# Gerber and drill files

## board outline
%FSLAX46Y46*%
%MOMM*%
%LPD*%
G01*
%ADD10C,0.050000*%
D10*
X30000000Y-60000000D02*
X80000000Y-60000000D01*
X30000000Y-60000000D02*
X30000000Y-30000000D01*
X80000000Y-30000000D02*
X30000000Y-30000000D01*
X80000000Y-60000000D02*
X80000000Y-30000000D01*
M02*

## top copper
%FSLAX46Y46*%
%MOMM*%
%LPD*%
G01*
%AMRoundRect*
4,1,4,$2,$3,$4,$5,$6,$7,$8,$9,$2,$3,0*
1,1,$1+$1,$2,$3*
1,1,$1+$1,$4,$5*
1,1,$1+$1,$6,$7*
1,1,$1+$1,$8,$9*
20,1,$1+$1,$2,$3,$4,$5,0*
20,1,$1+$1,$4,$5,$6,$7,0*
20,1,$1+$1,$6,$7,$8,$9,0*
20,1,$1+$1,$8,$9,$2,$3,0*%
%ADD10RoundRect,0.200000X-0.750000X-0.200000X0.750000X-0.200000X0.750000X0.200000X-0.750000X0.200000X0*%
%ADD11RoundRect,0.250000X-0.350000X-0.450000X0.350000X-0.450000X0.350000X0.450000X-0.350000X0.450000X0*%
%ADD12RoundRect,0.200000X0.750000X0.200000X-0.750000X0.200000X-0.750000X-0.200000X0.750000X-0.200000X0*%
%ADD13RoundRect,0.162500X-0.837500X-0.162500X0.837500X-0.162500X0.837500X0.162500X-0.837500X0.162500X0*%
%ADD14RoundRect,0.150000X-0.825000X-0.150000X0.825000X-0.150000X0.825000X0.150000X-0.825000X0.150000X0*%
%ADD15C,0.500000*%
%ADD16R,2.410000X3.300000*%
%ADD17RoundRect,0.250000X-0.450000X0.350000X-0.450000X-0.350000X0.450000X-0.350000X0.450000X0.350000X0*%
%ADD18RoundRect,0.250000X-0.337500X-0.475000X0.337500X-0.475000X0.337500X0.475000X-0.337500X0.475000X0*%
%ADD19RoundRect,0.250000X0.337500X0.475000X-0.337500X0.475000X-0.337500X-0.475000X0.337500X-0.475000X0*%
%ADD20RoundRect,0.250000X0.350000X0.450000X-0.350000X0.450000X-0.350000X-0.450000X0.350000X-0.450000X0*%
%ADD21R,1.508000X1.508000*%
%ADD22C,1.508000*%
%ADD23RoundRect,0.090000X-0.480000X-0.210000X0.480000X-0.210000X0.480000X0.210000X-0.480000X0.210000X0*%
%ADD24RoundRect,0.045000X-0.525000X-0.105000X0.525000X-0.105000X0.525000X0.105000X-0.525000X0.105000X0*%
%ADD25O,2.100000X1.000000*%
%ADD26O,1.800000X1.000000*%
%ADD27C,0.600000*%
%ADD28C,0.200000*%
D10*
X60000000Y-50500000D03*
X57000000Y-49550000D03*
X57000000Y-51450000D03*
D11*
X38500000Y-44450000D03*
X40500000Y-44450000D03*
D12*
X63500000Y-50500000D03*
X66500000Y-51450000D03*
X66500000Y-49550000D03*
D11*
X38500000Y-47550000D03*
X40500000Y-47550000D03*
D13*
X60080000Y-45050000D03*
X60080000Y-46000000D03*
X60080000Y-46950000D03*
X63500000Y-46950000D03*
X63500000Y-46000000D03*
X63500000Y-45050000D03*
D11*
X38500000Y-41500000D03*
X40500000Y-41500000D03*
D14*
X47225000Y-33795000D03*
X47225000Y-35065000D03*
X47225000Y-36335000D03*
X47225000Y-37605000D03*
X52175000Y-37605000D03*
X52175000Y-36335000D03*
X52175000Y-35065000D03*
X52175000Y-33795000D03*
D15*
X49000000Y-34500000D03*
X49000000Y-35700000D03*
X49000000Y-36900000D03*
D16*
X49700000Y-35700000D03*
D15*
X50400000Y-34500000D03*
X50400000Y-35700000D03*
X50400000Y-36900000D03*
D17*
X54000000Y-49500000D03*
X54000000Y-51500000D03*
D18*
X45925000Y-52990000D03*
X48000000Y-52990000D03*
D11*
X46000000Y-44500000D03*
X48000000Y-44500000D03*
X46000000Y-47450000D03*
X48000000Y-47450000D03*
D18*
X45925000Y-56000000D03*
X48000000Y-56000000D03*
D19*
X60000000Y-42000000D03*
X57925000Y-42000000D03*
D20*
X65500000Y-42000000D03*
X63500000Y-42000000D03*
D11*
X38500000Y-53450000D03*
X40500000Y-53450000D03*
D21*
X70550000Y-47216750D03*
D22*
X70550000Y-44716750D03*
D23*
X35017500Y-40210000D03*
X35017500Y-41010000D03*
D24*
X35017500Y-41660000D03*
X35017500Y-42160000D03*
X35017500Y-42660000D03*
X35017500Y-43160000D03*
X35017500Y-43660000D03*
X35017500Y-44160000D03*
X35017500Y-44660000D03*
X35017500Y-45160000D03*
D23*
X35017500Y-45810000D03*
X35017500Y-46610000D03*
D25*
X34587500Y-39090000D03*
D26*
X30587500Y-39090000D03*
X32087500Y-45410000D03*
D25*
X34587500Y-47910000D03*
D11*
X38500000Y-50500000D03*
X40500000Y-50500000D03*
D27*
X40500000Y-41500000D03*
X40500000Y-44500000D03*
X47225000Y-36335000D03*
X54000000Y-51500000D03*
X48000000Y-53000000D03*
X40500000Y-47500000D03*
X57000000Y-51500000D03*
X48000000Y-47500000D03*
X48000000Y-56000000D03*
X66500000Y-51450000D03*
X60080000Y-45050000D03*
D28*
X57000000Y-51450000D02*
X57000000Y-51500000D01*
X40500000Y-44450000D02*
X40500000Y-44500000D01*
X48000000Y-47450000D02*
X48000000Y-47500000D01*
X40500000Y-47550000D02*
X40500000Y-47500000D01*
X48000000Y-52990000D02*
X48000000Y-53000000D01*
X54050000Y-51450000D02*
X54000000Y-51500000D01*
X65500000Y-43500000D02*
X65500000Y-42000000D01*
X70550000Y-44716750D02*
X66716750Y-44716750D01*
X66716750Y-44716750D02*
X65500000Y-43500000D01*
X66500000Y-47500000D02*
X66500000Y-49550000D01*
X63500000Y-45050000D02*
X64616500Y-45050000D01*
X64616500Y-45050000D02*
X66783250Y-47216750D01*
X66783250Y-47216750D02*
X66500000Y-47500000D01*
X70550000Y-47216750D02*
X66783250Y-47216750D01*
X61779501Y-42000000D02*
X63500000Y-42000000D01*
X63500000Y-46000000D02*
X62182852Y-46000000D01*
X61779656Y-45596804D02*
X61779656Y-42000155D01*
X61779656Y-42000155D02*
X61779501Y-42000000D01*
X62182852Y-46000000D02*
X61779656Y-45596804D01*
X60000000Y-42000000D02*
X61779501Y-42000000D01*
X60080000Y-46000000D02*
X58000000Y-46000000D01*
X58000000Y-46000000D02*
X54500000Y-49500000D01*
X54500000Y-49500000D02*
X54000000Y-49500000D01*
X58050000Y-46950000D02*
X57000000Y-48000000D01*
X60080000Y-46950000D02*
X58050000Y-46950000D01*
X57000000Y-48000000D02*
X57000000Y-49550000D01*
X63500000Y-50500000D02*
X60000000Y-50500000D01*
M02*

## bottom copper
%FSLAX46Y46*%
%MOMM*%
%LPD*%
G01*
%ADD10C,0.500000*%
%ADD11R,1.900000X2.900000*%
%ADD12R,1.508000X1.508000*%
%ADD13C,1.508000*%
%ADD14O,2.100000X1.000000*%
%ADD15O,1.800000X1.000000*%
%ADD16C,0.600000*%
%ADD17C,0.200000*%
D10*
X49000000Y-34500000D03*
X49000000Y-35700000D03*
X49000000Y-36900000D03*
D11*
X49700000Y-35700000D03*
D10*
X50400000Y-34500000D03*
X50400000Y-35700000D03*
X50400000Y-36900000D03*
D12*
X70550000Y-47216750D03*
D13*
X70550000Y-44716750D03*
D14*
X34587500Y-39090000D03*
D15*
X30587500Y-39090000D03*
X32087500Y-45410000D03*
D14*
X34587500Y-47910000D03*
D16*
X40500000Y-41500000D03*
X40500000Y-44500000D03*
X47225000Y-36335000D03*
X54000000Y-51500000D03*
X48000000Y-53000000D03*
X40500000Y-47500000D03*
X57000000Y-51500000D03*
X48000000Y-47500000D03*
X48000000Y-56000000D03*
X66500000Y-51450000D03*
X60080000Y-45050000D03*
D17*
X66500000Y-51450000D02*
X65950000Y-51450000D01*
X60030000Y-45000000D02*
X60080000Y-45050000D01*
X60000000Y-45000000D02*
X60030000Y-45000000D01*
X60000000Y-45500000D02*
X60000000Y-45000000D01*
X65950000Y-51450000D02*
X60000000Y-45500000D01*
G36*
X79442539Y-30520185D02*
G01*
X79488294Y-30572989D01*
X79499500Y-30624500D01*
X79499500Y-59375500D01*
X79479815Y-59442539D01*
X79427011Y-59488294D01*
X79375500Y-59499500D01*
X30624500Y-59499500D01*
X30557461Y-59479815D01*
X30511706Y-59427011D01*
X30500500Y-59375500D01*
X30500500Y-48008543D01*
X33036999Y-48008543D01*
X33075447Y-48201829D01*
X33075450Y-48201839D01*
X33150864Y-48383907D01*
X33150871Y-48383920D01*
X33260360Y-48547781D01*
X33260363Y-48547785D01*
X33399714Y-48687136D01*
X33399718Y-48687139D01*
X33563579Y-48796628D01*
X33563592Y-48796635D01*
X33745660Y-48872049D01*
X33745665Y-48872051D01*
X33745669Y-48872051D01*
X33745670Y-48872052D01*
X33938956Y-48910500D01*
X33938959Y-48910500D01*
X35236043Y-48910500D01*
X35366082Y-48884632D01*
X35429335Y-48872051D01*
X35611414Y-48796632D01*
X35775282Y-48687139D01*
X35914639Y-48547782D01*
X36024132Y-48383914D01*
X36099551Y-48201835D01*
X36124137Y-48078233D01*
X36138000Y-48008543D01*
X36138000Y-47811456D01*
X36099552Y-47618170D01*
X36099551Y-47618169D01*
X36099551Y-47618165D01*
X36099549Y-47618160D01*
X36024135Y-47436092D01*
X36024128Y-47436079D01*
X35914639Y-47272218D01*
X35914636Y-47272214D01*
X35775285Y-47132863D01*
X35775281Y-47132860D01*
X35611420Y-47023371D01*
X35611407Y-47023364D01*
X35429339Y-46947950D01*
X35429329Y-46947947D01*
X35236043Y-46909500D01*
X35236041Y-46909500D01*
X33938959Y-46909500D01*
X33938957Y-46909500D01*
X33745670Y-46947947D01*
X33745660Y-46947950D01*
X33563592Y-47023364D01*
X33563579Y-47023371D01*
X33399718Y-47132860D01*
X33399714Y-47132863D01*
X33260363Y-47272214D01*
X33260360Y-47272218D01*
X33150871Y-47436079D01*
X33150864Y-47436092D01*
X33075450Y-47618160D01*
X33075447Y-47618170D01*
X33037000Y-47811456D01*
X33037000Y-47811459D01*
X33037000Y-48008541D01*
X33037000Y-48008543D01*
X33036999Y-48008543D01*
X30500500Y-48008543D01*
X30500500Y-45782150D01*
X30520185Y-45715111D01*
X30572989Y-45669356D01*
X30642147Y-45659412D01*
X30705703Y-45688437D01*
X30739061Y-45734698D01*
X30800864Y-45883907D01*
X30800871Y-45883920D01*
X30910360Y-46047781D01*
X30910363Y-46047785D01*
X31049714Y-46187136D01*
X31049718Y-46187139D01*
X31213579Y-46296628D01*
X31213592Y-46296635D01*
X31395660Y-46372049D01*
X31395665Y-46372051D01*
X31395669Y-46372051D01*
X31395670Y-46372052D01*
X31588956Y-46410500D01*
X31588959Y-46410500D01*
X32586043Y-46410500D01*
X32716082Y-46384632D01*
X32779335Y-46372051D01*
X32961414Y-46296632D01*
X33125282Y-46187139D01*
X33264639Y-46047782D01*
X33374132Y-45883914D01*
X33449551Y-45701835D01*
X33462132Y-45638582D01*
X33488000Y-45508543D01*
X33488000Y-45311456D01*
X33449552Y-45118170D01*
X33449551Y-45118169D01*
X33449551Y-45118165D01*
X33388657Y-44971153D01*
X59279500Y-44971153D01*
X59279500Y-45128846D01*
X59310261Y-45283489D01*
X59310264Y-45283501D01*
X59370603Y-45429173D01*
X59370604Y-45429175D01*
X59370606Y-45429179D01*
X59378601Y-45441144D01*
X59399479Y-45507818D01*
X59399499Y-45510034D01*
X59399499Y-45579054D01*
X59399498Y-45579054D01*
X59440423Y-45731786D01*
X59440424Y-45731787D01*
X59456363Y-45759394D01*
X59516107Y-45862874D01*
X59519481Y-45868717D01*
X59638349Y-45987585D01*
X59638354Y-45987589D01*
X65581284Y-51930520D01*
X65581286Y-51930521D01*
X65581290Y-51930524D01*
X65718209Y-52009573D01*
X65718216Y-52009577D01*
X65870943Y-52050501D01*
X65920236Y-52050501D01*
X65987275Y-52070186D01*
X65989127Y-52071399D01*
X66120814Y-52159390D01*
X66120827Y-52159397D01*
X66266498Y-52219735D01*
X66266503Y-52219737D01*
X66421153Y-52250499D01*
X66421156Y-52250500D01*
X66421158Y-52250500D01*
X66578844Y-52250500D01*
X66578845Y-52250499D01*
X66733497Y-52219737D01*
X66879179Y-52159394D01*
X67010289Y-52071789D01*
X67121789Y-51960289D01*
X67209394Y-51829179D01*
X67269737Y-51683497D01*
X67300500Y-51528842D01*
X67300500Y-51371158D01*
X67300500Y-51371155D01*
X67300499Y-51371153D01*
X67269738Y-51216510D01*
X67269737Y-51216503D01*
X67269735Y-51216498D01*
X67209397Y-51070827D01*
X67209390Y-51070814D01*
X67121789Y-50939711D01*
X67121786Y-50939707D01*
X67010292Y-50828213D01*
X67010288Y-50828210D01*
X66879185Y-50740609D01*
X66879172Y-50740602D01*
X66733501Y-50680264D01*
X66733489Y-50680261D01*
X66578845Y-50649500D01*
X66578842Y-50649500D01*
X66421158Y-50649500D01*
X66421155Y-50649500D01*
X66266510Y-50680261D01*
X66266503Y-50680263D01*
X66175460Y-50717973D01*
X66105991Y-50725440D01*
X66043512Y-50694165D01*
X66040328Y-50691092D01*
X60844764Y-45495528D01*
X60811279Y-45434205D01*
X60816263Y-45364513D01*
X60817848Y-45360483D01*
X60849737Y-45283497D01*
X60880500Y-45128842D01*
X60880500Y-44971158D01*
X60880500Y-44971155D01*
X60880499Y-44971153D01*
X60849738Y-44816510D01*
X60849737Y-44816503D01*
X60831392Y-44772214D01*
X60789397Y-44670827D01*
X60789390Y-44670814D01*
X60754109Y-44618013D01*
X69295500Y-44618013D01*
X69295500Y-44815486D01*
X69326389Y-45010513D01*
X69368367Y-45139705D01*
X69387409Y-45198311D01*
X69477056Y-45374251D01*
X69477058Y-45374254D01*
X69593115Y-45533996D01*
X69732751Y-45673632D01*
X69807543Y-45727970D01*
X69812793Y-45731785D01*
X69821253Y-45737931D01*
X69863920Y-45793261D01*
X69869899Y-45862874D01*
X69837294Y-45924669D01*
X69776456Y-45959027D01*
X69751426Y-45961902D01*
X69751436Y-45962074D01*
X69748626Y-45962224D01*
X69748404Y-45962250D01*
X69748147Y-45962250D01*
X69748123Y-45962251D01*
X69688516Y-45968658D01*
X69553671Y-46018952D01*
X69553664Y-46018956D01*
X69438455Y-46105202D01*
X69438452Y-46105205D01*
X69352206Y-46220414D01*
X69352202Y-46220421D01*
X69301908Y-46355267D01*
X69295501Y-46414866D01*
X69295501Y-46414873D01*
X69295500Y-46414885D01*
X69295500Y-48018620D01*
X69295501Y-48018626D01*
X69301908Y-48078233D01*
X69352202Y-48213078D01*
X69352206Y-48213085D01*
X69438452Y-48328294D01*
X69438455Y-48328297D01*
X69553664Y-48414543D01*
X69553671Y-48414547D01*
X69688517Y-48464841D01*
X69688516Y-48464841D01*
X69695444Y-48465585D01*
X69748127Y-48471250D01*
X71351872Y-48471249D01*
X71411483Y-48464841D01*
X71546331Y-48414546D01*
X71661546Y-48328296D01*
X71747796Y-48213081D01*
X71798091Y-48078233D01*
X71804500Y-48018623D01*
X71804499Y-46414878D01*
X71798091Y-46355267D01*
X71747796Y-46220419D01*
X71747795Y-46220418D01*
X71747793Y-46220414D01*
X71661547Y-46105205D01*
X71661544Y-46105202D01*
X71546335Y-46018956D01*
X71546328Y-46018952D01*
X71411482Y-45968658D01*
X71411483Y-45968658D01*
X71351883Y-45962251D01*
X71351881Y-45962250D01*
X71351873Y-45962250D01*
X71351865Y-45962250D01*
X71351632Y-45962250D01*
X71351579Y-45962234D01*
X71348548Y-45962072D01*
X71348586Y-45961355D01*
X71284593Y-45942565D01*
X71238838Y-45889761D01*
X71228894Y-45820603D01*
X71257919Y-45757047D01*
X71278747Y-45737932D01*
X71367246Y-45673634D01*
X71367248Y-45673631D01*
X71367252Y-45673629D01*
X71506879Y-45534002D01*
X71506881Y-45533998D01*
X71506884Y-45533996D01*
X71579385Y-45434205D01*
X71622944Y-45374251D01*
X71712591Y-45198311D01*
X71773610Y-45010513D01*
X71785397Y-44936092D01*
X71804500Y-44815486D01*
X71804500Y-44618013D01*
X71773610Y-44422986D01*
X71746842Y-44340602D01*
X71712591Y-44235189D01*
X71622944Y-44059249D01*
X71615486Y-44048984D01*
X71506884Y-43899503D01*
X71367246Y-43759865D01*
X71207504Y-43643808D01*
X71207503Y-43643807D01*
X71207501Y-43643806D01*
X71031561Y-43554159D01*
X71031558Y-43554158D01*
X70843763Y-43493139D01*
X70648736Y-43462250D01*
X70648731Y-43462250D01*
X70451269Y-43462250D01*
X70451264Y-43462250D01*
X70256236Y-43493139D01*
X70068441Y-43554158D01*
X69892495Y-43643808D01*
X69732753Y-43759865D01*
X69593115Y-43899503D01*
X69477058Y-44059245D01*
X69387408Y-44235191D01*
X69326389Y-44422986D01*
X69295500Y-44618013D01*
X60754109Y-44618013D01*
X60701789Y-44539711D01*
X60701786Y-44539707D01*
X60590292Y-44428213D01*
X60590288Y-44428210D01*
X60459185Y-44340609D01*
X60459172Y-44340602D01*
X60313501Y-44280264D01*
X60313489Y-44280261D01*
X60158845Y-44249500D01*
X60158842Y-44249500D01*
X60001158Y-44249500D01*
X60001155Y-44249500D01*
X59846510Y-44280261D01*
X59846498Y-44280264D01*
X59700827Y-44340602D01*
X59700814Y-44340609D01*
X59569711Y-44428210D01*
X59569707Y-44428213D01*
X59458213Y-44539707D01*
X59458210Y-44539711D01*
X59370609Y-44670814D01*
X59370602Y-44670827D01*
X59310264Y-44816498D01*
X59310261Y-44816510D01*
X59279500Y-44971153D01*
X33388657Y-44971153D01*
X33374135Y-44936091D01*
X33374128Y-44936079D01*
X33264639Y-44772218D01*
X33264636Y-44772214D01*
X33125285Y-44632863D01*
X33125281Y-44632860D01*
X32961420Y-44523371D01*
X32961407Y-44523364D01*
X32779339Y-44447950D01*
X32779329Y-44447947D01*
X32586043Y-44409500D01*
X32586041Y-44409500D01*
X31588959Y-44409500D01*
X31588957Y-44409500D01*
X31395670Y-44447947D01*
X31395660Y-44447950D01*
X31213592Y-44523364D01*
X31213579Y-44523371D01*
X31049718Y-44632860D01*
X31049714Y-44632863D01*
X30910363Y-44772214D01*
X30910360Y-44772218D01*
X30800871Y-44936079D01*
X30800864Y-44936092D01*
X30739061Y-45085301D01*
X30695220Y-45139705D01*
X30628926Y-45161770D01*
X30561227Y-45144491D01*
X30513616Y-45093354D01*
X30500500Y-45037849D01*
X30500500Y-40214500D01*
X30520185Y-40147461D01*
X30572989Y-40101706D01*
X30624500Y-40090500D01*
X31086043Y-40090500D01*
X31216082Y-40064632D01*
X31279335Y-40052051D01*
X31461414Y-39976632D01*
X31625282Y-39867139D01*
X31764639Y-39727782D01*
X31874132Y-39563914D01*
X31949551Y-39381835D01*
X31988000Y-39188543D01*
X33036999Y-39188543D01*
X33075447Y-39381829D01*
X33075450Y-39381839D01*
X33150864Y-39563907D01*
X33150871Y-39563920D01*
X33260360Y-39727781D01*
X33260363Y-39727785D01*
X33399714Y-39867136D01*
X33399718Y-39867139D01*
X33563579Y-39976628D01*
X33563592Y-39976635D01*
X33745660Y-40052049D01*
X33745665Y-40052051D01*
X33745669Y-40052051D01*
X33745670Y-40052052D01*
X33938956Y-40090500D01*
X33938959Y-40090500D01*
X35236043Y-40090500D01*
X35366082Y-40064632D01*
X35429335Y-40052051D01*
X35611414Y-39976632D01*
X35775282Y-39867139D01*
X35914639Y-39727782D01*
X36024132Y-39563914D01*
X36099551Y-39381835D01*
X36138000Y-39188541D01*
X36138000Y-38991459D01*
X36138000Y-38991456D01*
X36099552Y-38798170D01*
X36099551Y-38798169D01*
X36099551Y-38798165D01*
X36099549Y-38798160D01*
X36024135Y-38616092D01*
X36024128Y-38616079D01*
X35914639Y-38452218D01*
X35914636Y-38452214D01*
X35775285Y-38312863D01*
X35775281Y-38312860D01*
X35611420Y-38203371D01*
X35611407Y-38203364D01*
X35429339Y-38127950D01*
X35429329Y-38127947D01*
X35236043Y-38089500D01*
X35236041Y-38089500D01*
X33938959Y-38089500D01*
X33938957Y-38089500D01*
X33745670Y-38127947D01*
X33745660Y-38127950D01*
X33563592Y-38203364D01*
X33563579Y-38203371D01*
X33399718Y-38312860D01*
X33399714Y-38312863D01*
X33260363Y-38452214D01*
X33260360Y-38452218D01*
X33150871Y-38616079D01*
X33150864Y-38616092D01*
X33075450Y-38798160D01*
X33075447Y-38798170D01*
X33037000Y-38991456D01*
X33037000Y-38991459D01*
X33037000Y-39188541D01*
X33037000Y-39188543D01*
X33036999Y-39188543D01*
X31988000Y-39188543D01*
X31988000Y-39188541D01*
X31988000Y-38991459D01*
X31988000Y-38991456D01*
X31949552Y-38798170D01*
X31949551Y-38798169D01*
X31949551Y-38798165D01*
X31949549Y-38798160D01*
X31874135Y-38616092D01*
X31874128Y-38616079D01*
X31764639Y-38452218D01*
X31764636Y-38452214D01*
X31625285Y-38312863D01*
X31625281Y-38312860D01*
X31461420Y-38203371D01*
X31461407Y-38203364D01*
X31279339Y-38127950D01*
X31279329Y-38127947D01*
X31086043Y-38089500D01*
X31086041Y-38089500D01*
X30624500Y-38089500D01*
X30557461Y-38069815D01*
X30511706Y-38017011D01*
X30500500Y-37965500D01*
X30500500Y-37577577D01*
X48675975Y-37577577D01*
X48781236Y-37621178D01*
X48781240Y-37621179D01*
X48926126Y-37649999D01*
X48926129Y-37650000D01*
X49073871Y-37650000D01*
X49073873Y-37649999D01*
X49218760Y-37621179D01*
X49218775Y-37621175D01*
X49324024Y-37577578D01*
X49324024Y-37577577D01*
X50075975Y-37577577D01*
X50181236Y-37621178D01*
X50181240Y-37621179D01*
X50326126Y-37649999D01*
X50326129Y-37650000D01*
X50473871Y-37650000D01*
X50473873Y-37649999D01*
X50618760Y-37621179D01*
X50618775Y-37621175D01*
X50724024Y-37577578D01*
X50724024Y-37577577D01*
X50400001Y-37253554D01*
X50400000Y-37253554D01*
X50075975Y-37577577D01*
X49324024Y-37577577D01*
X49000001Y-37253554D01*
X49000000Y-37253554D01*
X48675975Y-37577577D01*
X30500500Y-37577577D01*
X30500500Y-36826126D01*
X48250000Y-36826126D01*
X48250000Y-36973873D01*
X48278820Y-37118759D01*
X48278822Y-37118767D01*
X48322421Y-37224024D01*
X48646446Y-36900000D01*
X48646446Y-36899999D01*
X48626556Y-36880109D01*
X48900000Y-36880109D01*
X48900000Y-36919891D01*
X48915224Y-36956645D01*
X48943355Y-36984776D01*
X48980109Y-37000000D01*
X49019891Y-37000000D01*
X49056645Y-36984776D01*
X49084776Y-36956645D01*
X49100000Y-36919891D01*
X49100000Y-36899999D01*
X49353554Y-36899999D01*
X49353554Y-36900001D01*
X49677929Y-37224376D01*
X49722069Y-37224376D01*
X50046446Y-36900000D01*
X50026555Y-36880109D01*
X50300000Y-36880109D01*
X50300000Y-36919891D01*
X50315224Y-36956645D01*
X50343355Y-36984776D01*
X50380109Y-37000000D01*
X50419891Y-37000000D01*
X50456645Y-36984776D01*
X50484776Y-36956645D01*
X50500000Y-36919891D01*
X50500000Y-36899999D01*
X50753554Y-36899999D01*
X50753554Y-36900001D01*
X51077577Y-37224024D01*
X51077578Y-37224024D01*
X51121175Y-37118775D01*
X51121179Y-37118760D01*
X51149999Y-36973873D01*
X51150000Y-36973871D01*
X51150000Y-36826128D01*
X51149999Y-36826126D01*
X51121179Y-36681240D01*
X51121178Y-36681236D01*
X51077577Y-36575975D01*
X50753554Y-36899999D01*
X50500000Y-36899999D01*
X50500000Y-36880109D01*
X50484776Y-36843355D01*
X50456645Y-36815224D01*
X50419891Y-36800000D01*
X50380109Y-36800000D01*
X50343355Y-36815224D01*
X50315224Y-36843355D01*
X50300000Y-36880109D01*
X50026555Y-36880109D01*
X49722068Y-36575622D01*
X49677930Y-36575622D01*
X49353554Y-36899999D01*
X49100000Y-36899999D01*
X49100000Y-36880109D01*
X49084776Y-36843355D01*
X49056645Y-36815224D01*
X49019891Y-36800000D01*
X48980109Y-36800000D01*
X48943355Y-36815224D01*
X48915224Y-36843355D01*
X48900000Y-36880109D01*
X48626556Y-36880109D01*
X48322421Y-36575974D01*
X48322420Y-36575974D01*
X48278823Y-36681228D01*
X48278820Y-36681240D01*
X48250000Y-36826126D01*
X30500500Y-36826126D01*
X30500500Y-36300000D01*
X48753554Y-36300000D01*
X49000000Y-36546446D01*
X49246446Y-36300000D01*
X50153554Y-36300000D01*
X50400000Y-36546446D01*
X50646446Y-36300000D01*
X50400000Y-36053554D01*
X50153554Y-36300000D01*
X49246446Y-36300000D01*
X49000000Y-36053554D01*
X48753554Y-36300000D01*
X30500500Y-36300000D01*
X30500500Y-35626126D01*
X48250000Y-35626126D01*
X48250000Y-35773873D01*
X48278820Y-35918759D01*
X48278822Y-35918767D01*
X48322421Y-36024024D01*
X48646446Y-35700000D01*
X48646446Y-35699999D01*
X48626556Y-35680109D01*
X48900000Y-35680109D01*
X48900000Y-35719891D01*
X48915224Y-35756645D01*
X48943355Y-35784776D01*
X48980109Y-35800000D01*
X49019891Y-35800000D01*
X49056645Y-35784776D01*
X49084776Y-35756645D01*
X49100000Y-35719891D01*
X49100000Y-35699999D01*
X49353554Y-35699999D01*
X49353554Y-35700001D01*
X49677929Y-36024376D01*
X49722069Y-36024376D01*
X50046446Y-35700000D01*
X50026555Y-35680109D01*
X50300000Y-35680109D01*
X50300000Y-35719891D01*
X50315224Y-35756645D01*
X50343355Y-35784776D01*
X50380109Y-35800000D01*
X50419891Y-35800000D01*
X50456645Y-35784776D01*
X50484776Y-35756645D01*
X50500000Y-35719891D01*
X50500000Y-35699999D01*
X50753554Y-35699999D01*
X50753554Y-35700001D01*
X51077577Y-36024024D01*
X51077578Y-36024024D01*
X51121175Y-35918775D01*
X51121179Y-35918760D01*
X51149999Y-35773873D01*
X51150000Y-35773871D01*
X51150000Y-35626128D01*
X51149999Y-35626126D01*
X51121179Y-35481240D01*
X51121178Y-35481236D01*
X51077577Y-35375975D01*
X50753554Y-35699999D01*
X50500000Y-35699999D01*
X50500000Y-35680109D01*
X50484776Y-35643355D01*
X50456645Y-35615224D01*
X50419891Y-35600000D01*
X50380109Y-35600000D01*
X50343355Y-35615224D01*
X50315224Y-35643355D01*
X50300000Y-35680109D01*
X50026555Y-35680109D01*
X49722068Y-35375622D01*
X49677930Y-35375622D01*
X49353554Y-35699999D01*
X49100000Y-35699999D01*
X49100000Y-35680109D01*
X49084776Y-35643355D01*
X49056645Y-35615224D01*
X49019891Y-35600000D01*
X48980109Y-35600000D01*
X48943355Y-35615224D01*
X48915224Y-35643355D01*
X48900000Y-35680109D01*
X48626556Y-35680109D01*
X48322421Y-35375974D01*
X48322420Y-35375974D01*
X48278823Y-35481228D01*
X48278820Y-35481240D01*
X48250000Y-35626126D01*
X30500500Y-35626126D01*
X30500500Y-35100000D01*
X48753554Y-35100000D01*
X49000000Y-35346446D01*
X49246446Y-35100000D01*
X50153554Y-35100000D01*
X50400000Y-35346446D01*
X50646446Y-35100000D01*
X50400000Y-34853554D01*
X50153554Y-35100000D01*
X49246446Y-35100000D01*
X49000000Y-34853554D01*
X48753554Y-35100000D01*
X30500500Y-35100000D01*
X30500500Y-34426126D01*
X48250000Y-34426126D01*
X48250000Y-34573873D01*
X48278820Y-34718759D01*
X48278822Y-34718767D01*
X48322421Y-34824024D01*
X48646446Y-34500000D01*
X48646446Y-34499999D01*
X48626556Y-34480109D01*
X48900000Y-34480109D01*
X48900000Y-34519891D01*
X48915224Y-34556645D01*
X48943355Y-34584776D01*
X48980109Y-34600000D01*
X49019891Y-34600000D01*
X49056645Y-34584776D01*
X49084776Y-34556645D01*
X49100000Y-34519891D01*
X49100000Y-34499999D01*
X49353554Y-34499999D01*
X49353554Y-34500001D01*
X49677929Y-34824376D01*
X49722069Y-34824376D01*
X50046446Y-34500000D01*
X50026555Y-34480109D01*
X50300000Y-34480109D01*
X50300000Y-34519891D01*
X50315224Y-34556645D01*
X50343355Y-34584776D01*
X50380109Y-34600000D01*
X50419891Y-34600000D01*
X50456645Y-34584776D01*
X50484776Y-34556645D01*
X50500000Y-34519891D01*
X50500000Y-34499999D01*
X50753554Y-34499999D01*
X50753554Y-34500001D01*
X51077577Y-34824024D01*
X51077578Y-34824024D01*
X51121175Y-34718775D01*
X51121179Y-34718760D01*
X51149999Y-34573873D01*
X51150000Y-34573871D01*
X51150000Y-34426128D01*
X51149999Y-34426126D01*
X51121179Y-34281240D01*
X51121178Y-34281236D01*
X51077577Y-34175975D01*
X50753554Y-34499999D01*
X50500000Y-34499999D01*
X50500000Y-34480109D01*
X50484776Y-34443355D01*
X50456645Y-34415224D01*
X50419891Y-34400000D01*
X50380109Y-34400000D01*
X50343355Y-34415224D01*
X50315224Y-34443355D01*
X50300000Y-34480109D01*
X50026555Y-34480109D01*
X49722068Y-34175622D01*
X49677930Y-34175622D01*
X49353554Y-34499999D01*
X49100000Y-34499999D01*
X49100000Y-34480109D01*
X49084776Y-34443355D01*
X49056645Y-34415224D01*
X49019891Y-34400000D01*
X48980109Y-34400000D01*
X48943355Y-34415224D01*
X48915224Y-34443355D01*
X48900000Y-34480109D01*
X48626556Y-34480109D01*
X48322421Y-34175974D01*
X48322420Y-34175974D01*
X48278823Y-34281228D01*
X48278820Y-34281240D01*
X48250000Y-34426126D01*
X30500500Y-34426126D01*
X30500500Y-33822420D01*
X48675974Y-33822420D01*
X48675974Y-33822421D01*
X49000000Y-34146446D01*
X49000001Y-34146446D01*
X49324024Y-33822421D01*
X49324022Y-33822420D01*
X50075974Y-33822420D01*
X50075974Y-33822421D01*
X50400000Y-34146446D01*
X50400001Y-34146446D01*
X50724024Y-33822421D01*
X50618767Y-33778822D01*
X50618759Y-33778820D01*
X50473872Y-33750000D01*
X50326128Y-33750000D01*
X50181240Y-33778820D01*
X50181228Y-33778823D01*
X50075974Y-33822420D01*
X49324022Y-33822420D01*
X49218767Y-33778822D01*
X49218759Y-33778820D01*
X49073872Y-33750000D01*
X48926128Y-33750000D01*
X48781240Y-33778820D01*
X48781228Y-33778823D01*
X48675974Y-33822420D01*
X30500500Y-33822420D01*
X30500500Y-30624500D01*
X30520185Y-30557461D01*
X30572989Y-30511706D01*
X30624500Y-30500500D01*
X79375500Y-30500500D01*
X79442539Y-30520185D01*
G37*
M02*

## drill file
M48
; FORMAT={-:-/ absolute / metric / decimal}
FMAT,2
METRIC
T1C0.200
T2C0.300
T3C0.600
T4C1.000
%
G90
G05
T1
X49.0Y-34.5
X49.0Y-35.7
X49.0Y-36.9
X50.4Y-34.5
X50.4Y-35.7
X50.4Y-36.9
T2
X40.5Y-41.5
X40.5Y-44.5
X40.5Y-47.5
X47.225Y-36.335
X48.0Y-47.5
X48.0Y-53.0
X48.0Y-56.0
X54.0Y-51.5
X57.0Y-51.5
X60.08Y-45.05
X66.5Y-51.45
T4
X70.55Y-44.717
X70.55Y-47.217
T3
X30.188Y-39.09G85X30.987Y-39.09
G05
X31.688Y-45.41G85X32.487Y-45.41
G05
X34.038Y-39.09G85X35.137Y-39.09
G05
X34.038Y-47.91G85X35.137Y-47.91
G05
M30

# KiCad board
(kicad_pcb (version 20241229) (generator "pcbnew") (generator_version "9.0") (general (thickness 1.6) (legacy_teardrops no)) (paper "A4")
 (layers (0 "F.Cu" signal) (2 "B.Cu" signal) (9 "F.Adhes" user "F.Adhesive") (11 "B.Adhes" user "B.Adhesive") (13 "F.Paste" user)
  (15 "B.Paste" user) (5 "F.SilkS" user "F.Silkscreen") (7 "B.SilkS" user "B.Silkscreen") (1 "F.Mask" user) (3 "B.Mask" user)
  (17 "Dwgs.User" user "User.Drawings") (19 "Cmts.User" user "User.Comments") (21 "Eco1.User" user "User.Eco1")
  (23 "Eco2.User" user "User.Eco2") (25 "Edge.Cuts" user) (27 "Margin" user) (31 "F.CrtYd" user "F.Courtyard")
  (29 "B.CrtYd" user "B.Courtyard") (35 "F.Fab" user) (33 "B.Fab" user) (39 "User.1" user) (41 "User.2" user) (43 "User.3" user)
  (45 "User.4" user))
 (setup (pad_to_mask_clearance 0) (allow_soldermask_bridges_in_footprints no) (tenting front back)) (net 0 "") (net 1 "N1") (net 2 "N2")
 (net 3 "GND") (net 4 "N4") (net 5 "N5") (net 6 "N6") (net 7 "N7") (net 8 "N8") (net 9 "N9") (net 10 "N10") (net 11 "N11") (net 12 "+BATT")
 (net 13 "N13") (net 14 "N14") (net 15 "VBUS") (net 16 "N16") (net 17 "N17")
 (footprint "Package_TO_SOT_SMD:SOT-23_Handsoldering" (layer "F.Cu") (at 58.5 50.5)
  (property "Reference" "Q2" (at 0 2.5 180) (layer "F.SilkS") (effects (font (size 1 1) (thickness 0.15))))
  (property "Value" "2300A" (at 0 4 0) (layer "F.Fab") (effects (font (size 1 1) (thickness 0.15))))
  (pad "1" smd roundrect (at 1.5 0) (size 1.9 0.8) (layers "F.Cu" "F.Mask" "F.Paste") (roundrect_rratio 0.25) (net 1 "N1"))
  (pad "2" smd roundrect (at -1.5 -0.95) (size 1.9 0.8) (layers "F.Cu" "F.Mask" "F.Paste") (roundrect_rratio 0.25) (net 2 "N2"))
  (pad "3" smd roundrect (at -1.5 0.95) (size 1.9 0.8) (layers "F.Cu" "F.Mask" "F.Paste") (roundrect_rratio 0.25) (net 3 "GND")))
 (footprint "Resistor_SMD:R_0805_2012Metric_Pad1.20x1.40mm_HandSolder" (layer "F.Cu") (at 39.5 44.45)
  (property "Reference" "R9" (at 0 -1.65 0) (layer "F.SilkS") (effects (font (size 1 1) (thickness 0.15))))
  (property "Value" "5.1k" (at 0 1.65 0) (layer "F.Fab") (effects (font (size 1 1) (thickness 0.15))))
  (pad "1" smd roundrect (at -1 0) (size 1.2 1.4) (layers "F.Cu" "F.Mask" "F.Paste") (roundrect_rratio 0.208333) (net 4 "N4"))
  (pad "2" smd roundrect (at 1 0) (size 1.2 1.4) (layers "F.Cu" "F.Mask" "F.Paste") (roundrect_rratio 0.208333) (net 3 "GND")))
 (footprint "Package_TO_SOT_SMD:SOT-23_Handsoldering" (layer "F.Cu") (at 65 50.5 180)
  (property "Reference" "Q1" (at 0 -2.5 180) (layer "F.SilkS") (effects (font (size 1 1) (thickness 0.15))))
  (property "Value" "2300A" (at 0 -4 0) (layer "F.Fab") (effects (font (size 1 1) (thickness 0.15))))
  (pad "1" smd roundrect (at 1.5 0 180) (size 1.9 0.8) (layers "F.Cu" "F.Mask" "F.Paste") (roundrect_rratio 0.25) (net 1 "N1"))
  (pad "2" smd roundrect (at -1.5 -0.95 180) (size 1.9 0.8) (layers "F.Cu" "F.Mask" "F.Paste") (roundrect_rratio 0.25) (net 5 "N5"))
  (pad "3" smd roundrect (at -1.5 0.95 180) (size 1.9 0.8) (layers "F.Cu" "F.Mask" "F.Paste") (roundrect_rratio 0.25) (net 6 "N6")))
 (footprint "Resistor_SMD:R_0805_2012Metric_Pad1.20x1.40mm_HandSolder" (layer "F.Cu") (at 39.5 47.55)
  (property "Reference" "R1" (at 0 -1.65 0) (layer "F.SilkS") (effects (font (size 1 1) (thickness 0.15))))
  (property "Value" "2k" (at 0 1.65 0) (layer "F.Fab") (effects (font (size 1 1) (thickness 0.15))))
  (pad "1" smd roundrect (at -1 0) (size 1.2 1.4) (layers "F.Cu" "F.Mask" "F.Paste") (roundrect_rratio 0.208333) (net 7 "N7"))
  (pad "2" smd roundrect (at 1 0) (size 1.2 1.4) (layers "F.Cu" "F.Mask" "F.Paste") (roundrect_rratio 0.208333) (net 3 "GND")))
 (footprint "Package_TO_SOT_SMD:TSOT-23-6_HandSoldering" (layer "F.Cu") (at 61.79 46)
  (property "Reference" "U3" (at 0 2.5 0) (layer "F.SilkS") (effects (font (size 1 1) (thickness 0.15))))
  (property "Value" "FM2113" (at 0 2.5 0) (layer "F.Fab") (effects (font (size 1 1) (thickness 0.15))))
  (pad "1" smd roundrect (at -1.71 -0.95) (size 2 0.65) (layers "F.Cu" "F.Mask" "F.Paste") (roundrect_rratio 0.25) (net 5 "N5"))
  (pad "2" smd roundrect (at -1.71 0) (size 2 0.65) (layers "F.Cu" "F.Mask" "F.Paste") (roundrect_rratio 0.25) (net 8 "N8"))
  (pad "3" smd roundrect (at -1.71 0.95) (size 2 0.65) (layers "F.Cu" "F.Mask" "F.Paste") (roundrect_rratio 0.25) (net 2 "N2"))
  (pad "4" smd roundrect (at 1.71 0.95) (size 2 0.65) (layers "F.Cu" "F.Mask" "F.Paste") (roundrect_rratio 0.25))
  (pad "5" smd roundrect (at 1.71 0) (size 2 0.65) (layers "F.Cu" "F.Mask" "F.Paste") (roundrect_rratio 0.25) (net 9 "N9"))
  (pad "6" smd roundrect (at 1.71 -0.95) (size 2 0.65) (layers "F.Cu" "F.Mask" "F.Paste") (roundrect_rratio 0.25) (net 6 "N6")))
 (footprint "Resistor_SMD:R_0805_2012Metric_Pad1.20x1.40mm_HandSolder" (layer "F.Cu") (at 39.5 41.5)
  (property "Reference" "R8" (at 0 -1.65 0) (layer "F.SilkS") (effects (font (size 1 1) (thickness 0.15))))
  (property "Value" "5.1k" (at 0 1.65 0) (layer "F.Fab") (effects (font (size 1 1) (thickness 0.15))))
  (pad "1" smd roundrect (at -1 0) (size 1.2 1.4) (layers "F.Cu" "F.Mask" "F.Paste") (roundrect_rratio 0.208333) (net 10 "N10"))
  (pad "2" smd roundrect (at 1 0) (size 1.2 1.4) (layers "F.Cu" "F.Mask" "F.Paste") (roundrect_rratio 0.208333) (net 3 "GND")))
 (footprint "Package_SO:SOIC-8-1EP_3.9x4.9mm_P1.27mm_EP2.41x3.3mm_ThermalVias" (layer "F.Cu") (at 49.7 35.7)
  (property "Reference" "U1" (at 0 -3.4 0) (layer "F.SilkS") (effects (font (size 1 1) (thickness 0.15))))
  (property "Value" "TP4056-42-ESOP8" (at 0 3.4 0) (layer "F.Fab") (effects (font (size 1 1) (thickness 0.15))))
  (pad "" smd roundrect (at -0.6 -0.825) (size 1.01 1.38) (layers "F.Paste") (roundrect_rratio 0.247525))
  (pad "" smd roundrect (at -0.6 0.825) (size 1.01 1.38) (layers "F.Paste") (roundrect_rratio 0.247525))
  (pad "" smd roundrect (at 0.6 -0.825) (size 1.01 1.38) (layers "F.Paste") (roundrect_rratio 0.247525))
  (pad "" smd roundrect (at 0.6 0.825) (size 1.01 1.38) (layers "F.Paste") (roundrect_rratio 0.247525))
  (pad "1" smd roundrect (at -2.475 -1.905) (size 1.95 0.6) (layers "F.Cu" "F.Mask" "F.Paste") (roundrect_rratio 0.25) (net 3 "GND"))
  (pad "2" smd roundrect (at -2.475 -0.635) (size 1.95 0.6) (layers "F.Cu" "F.Mask" "F.Paste") (roundrect_rratio 0.25) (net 7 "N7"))
  (pad "3" smd roundrect (at -2.475 0.635) (size 1.95 0.6) (layers "F.Cu" "F.Mask" "F.Paste") (roundrect_rratio 0.25) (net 3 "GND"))
  (pad "4" smd roundrect (at -2.475 1.905) (size 1.95 0.6) (layers "F.Cu" "F.Mask" "F.Paste") (roundrect_rratio 0.25) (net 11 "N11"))
  (pad "5" smd roundrect (at 2.475 1.905) (size 1.95 0.6) (layers "F.Cu" "F.Mask" "F.Paste") (roundrect_rratio 0.25) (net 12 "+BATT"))
  (pad "6" smd roundrect (at 2.475 0.635) (size 1.95 0.6) (layers "F.Cu" "F.Mask" "F.Paste") (roundrect_rratio 0.25) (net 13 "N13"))
  (pad "7" smd roundrect (at 2.475 -0.635) (size 1.95 0.6) (layers "F.Cu" "F.Mask" "F.Paste") (roundrect_rratio 0.25) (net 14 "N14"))
  (pad "8" smd roundrect (at 2.475 -1.905) (size 1.95 0.6) (layers "F.Cu" "F.Mask" "F.Paste") (roundrect_rratio 0.25) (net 11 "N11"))
  (pad "9" thru_hole circle (at -0.7 -1.2) (size 0.5 0.5) (drill 0.2) (layers "*.Cu") (remove_unused_layers no) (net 3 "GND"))
  (pad "9" thru_hole circle (at -0.7 0) (size 0.5 0.5) (drill 0.2) (layers "*.Cu") (remove_unused_layers no) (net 3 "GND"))
  (pad "9" thru_hole circle (at -0.7 1.2) (size 0.5 0.5) (drill 0.2) (layers "*.Cu") (remove_unused_layers no) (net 3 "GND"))
  (pad "9" smd rect (at 0 0) (size 1.9 2.9) (layers "B.Cu") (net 3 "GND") (zone_connect 2))
  (pad "9" smd rect (at 0 0) (size 2.41 3.3) (layers "F.Cu" "F.Mask") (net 3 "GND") (zone_connect 2))
  (pad "9" thru_hole circle (at 0.7 -1.2) (size 0.5 0.5) (drill 0.2) (layers "*.Cu") (remove_unused_layers no) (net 3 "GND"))
  (pad "9" thru_hole circle (at 0.7 0) (size 0.5 0.5) (drill 0.2) (layers "*.Cu") (remove_unused_layers no) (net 3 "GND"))
  (pad "9" thru_hole circle (at 0.7 1.2) (size 0.5 0.5) (drill 0.2) (layers "*.Cu") (remove_unused_layers no) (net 3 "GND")))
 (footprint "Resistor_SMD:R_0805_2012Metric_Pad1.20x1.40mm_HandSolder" (layer "F.Cu") (at 54 50.5 -90)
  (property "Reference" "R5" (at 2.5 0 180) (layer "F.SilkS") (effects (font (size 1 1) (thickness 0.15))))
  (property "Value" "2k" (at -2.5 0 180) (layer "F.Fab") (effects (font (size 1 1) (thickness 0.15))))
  (pad "1" smd roundrect (at -1 0 270) (size 1.2 1.4) (layers "F.Cu" "F.Mask" "F.Paste") (roundrect_rratio 0.208333) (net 8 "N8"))
  (pad "2" smd roundrect (at 1 0 270) (size 1.2 1.4) (layers "F.Cu" "F.Mask" "F.Paste") (roundrect_rratio 0.208333) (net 3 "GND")))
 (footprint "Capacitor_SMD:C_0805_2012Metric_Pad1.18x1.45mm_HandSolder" (layer "F.Cu") (at 46.9625 52.99)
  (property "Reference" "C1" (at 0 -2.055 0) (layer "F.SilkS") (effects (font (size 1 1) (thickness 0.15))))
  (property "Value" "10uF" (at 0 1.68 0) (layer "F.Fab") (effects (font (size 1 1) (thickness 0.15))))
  (pad "1" smd roundrect (at -1.0375 0) (size 1.175 1.45) (layers "F.Cu" "F.Mask" "F.Paste") (roundrect_rratio 0.212766) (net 11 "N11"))
  (pad "2" smd roundrect (at 1.0375 0) (size 1.175 1.45) (layers "F.Cu" "F.Mask" "F.Paste") (roundrect_rratio 0.212766) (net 3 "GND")))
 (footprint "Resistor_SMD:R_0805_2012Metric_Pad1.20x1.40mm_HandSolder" (layer "F.Cu") (at 47 44.5)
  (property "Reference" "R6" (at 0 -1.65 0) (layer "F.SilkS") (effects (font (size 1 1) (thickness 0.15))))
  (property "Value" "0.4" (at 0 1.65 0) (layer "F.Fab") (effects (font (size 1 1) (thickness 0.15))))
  (pad "1" smd roundrect (at -1 0) (size 1.2 1.4) (layers "F.Cu" "F.Mask" "F.Paste") (roundrect_rratio 0.208333) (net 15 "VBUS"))
  (pad "2" smd roundrect (at 1 0) (size 1.2 1.4) (layers "F.Cu" "F.Mask" "F.Paste") (roundrect_rratio 0.208333) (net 11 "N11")))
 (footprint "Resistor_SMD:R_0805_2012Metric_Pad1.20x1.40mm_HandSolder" (layer "F.Cu") (at 47 47.45)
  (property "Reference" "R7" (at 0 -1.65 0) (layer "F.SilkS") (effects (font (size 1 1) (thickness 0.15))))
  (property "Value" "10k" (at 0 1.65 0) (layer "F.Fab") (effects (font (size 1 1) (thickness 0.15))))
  (pad "1" smd roundrect (at -1 0) (size 1.2 1.4) (layers "F.Cu" "F.Mask" "F.Paste") (roundrect_rratio 0.208333) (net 11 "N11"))
  (pad "2" smd roundrect (at 1 0) (size 1.2 1.4) (layers "F.Cu" "F.Mask" "F.Paste") (roundrect_rratio 0.208333) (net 3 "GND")))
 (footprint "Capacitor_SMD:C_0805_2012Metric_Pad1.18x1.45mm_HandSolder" (layer "F.Cu") (at 46.9625 56)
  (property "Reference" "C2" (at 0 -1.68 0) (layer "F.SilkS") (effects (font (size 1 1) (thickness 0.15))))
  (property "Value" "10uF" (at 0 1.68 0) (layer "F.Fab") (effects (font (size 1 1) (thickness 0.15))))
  (pad "1" smd roundrect (at -1.0375 0) (size 1.175 1.45) (layers "F.Cu" "F.Mask" "F.Paste") (roundrect_rratio 0.212766) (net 12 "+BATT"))
  (pad "2" smd roundrect (at 1.0375 0) (size 1.175 1.45) (layers "F.Cu" "F.Mask" "F.Paste") (roundrect_rratio 0.212766) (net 3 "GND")))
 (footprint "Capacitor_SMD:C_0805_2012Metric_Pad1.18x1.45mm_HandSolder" (layer "F.Cu") (at 58.9625 42 180)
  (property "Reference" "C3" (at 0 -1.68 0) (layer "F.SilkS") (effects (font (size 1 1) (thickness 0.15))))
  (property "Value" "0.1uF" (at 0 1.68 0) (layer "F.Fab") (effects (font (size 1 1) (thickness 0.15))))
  (pad "1" smd roundrect (at -1.0375 0 180) (size 1.175 1.45) (layers "F.Cu" "F.Mask" "F.Paste") (roundrect_rratio 0.212766) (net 9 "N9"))
  (pad "2" smd roundrect (at 1.0375 0 180) (size 1.175 1.45) (layers "F.Cu" "F.Mask" "F.Paste") (roundrect_rratio 0.212766) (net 6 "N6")))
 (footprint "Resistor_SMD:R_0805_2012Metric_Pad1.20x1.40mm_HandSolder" (layer "F.Cu") (at 64.5 42 180)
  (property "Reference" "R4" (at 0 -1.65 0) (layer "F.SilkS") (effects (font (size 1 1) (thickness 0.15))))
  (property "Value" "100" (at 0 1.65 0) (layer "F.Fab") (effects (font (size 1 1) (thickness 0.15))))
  (pad "1" smd roundrect (at -1 0 180) (size 1.2 1.4) (layers "F.Cu" "F.Mask" "F.Paste") (roundrect_rratio 0.208333) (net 12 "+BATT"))
  (pad "2" smd roundrect (at 1 0 180) (size 1.2 1.4) (layers "F.Cu" "F.Mask" "F.Paste") (roundrect_rratio 0.208333) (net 9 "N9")))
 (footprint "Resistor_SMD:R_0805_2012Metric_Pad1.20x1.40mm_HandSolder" (layer "F.Cu") (at 39.5 53.45)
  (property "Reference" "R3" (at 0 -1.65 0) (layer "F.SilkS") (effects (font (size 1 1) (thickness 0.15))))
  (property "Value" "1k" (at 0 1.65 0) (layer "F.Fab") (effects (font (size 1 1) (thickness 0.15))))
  (pad "1" smd roundrect (at -1 0) (size 1.2 1.4) (layers "F.Cu" "F.Mask" "F.Paste") (roundrect_rratio 0.208333) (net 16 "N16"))
  (pad "2" smd roundrect (at 1 0) (size 1.2 1.4) (layers "F.Cu" "F.Mask" "F.Paste") (roundrect_rratio 0.208333) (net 13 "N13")))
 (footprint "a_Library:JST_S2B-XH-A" (layer "F.Cu") (at 76.25 45.96675 90)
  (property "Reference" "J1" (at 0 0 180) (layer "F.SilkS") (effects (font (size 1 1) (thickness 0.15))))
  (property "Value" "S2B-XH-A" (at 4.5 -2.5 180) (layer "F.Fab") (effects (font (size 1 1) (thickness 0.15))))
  (pad "1" thru_hole rect (at -1.25 -5.7 90) (size 1.508 1.508) (drill 1) (layers "*.Cu" "*.Mask") (remove_unused_layers no) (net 6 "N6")
   (solder_mask_margin 0.102))
  (pad "2" thru_hole circle (at 1.25 -5.7 90) (size 1.508 1.508) (drill 1) (layers "*.Cu" "*.Mask") (remove_unused_layers no)
   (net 12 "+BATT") (solder_mask_margin 0.102)))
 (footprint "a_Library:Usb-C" (layer "F.Cu") (at 35.5875 43.41 -90)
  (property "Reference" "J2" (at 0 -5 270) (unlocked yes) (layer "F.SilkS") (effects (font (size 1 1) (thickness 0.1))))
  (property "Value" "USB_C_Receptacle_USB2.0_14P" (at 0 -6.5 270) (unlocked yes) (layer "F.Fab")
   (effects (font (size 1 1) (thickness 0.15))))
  (pad "" smd roundrect (at -3.2 0.57) (size 1.14 0.6) (layers "F.Cu" "F.Mask" "F.Paste") (roundrect_rratio 0.15) (thermal_bridge_angle 45))
  (pad "" smd roundrect (at -2.4 0.57) (size 1.14 0.6) (layers "F.Cu" "F.Mask" "F.Paste") (roundrect_rratio 0.15) (thermal_bridge_angle 45))
  (pad "" smd roundrect (at -1.75 0.57) (size 1.14 0.3) (layers "F.Cu" "F.Mask" "F.Paste") (roundrect_rratio 0.15) (thermal_bridge_angle 45))
  (pad "" smd roundrect (at -1.25 0.57) (size 1.14 0.3) (layers "F.Cu" "F.Mask" "F.Paste") (roundrect_rratio 0.15) (thermal_bridge_angle 45))
  (pad "" smd roundrect (at -0.75 0.57) (size 1.14 0.3) (layers "F.Cu" "F.Mask" "F.Paste") (roundrect_rratio 0.15) (thermal_bridge_angle 45))
  (pad "" smd roundrect (at -0.25 0.57) (size 1.14 0.3) (layers "F.Cu" "F.Mask" "F.Paste") (roundrect_rratio 0.15) (thermal_bridge_angle 45))
  (pad "" smd roundrect (at 0.25 0.57) (size 1.14 0.3) (layers "F.Cu" "F.Mask" "F.Paste") (roundrect_rratio 0.15) (thermal_bridge_angle 45))
  (pad "" smd roundrect (at 0.75 0.57) (size 1.14 0.3) (layers "F.Cu" "F.Mask" "F.Paste") (roundrect_rratio 0.15) (thermal_bridge_angle 45))
  (pad "" smd roundrect (at 1.25 0.57) (size 1.14 0.3) (layers "F.Cu" "F.Mask" "F.Paste") (roundrect_rratio 0.15) (thermal_bridge_angle 45))
  (pad "" smd roundrect (at 1.75 0.57) (size 1.14 0.3) (layers "F.Cu" "F.Mask" "F.Paste") (roundrect_rratio 0.15) (thermal_bridge_angle 45))
  (pad "" smd roundrect (at 2.4 0.57) (size 1.14 0.6) (layers "F.Cu" "F.Mask" "F.Paste") (roundrect_rratio 0.15) (thermal_bridge_angle 45))
  (pad "" smd roundrect (at 3.2 0.57) (size 1.14 0.6) (layers "F.Cu" "F.Mask" "F.Paste") (roundrect_rratio 0.15) (thermal_bridge_angle 45))
  (pad "7" thru_hole oval (at -4.32 1) (size 2.1 1) (drill oval 1.7 0.6) (layers "*.Cu" "*.Mask") (remove_unused_layers no)
   (thermal_bridge_angle 45))
  (pad "7" thru_hole oval (at -4.32 5) (size 1.8 1) (drill oval 1.4 0.6) (layers "*.Cu" "*.Mask") (remove_unused_layers no)
   (thermal_bridge_angle 45))
  (pad "7" thru_hole oval (at 2 3.5) (size 1.8 1) (drill oval 1.4 0.6) (layers "*.Cu" "*.Mask") (remove_unused_layers no)
   (thermal_bridge_angle 45))
  (pad "7" thru_hole oval (at 4.5 1) (size 2.1 1) (drill oval 1.7 0.6) (layers "*.Cu" "*.Mask") (remove_unused_layers no)
   (thermal_bridge_angle 45)))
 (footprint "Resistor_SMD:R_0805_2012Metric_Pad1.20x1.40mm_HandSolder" (layer "F.Cu") (at 39.5 50.5)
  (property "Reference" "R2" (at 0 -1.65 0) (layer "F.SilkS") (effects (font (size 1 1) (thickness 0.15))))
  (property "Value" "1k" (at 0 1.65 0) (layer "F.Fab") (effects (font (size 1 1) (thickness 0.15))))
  (pad "1" smd roundrect (at -1 0) (size 1.2 1.4) (layers "F.Cu" "F.Mask" "F.Paste") (roundrect_rratio 0.208333) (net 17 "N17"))
  (pad "2" smd roundrect (at 1 0) (size 1.2 1.4) (layers "F.Cu" "F.Mask" "F.Paste") (roundrect_rratio 0.208333) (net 14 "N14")))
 (gr_line (start 30 60) (end 80 60) (stroke (width 0.05) (type default)) (layer "Edge.Cuts"))
 (gr_line (start 30 60) (end 30 30) (stroke (width 0.05) (type solid)) (layer "Edge.Cuts"))
 (gr_line (start 80 30) (end 30 30) (stroke (width 0.05) (type default)) (layer "Edge.Cuts"))
 (gr_line (start 80 60) (end 80 30) (stroke (width 0.05) (type solid)) (layer "Edge.Cuts"))
 (segment (start 57 51.45) (end 57 51.5) (width 0.2) (layer "F.Cu") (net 3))
 (segment (start 40.5 44.45) (end 40.5 44.5) (width 0.2) (layer "F.Cu") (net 3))
 (segment (start 48 47.45) (end 48 47.5) (width 0.2) (layer "F.Cu") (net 3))
 (segment (start 40.5 47.55) (end 40.5 47.5) (width 0.2) (layer "F.Cu") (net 3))
 (segment (start 48 52.99) (end 48 53) (width 0.2) (layer "F.Cu") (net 3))
 (segment (start 54.05 51.45) (end 54 51.5) (width 0.2) (layer "F.Cu") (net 3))
 (via (at 40.5 41.5) (size 0.6) (drill 0.3) (layers "F.Cu" "B.Cu") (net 3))
 (via (at 40.5 44.5) (size 0.6) (drill 0.3) (layers "F.Cu" "B.Cu") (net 3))
 (via (at 47.225 36.335) (size 0.6) (drill 0.3) (layers "F.Cu" "B.Cu") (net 3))
 (via (at 54 51.5) (size 0.6) (drill 0.3) (layers "F.Cu" "B.Cu") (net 3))
 (via (at 48 53) (size 0.6) (drill 0.3) (layers "F.Cu" "B.Cu") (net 3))
 (via (at 40.5 47.5) (size 0.6) (drill 0.3) (layers "F.Cu" "B.Cu") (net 3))
 (via (at 57 51.5) (size 0.6) (drill 0.3) (layers "F.Cu" "B.Cu") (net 3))
 (via (at 48 47.5) (size 0.6) (drill 0.3) (layers "F.Cu" "B.Cu") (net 3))
 (via (at 48 56) (size 0.6) (drill 0.3) (layers "F.Cu" "B.Cu") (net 3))
 (segment (start 65.5 43.5) (end 65.5 42) (width 0.2) (layer "F.Cu") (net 12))
 (segment (start 70.55 44.71675) (end 66.71675 44.71675) (width 0.2) (layer "F.Cu") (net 12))
 (segment (start 66.71675 44.71675) (end 65.5 43.5) (width 0.2) (layer "F.Cu") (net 12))
 (segment (start 66.5 47.5) (end 66.5 49.55) (width 0.2) (layer "F.Cu") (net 6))
 (segment (start 63.5 45.05) (end 64.6165 45.05) (width 0.2) (layer "F.Cu") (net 6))
 (segment (start 64.6165 45.05) (end 66.78325 47.21675) (width 0.2) (layer "F.Cu") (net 6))
 (segment (start 66.78325 47.21675) (end 66.5 47.5) (width 0.2) (layer "F.Cu") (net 6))
 (segment (start 70.55 47.21675) (end 66.78325 47.21675) (width 0.2) (layer "F.Cu") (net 6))
 (via (at 66.5 51.45) (size 0.6) (drill 0.3) (layers "F.Cu" "B.Cu") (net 5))
 (via (at 60.08 45.05) (size 0.6) (drill 0.3) (layers "F.Cu" "B.Cu") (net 5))
 (segment (start 66.5 51.45) (end 65.95 51.45) (width 0.2) (layer "B.Cu") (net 5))
 (segment (start 60.03 45) (end 60.08 45.05) (width 0.2) (layer "B.Cu") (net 5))
 (segment (start 60 45) (end 60.03 45) (width 0.2) (layer "B.Cu") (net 5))
 (segment (start 60 45.5) (end 60 45) (width 0.2) (layer "B.Cu") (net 5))
 (segment (start 65.95 51.45) (end 60 45.5) (width 0.2) (layer "B.Cu") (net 5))
 (segment (start 61.779501 42) (end 63.5 42) (width 0.2) (layer "F.Cu") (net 9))
 (segment (start 63.5 46) (end 62.182852 46) (width 0.2) (layer "F.Cu") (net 9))
 (segment (start 61.779656 45.596804) (end 61.779656 42.000155) (width 0.2) (layer "F.Cu") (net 9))
 (segment (start 61.779656 42.000155) (end 61.779501 42) (width 0.2) (layer "F.Cu") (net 9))
 (segment (start 62.182852 46) (end 61.779656 45.596804) (width 0.2) (layer "F.Cu") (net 9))
 (segment (start 60 42) (end 61.779501 42) (width 0.2) (layer "F.Cu") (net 9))
 (segment (start 60.08 46) (end 58 46) (width 0.2) (layer "F.Cu") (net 8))
 (segment (start 58 46) (end 54.5 49.5) (width 0.2) (layer "F.Cu") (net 8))
 (segment (start 54.5 49.5) (end 54 49.5) (width 0.2) (layer "F.Cu") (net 8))
 (segment (start 58.05 46.95) (end 57 48) (width 0.2) (layer "F.Cu") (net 2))
 (segment (start 60.08 46.95) (end 58.05 46.95) (width 0.2) (layer "F.Cu") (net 2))
 (segment (start 57 48) (end 57 49.55) (width 0.2) (layer "F.Cu") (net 2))
 (segment (start 63.5 50.5) (end 60 50.5) (width 0.2) (layer "F.Cu") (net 1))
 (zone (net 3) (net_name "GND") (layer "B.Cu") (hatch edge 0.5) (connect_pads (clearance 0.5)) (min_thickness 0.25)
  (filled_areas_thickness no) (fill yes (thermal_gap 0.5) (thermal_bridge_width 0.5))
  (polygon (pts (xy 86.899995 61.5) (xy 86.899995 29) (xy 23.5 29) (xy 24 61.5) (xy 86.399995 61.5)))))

